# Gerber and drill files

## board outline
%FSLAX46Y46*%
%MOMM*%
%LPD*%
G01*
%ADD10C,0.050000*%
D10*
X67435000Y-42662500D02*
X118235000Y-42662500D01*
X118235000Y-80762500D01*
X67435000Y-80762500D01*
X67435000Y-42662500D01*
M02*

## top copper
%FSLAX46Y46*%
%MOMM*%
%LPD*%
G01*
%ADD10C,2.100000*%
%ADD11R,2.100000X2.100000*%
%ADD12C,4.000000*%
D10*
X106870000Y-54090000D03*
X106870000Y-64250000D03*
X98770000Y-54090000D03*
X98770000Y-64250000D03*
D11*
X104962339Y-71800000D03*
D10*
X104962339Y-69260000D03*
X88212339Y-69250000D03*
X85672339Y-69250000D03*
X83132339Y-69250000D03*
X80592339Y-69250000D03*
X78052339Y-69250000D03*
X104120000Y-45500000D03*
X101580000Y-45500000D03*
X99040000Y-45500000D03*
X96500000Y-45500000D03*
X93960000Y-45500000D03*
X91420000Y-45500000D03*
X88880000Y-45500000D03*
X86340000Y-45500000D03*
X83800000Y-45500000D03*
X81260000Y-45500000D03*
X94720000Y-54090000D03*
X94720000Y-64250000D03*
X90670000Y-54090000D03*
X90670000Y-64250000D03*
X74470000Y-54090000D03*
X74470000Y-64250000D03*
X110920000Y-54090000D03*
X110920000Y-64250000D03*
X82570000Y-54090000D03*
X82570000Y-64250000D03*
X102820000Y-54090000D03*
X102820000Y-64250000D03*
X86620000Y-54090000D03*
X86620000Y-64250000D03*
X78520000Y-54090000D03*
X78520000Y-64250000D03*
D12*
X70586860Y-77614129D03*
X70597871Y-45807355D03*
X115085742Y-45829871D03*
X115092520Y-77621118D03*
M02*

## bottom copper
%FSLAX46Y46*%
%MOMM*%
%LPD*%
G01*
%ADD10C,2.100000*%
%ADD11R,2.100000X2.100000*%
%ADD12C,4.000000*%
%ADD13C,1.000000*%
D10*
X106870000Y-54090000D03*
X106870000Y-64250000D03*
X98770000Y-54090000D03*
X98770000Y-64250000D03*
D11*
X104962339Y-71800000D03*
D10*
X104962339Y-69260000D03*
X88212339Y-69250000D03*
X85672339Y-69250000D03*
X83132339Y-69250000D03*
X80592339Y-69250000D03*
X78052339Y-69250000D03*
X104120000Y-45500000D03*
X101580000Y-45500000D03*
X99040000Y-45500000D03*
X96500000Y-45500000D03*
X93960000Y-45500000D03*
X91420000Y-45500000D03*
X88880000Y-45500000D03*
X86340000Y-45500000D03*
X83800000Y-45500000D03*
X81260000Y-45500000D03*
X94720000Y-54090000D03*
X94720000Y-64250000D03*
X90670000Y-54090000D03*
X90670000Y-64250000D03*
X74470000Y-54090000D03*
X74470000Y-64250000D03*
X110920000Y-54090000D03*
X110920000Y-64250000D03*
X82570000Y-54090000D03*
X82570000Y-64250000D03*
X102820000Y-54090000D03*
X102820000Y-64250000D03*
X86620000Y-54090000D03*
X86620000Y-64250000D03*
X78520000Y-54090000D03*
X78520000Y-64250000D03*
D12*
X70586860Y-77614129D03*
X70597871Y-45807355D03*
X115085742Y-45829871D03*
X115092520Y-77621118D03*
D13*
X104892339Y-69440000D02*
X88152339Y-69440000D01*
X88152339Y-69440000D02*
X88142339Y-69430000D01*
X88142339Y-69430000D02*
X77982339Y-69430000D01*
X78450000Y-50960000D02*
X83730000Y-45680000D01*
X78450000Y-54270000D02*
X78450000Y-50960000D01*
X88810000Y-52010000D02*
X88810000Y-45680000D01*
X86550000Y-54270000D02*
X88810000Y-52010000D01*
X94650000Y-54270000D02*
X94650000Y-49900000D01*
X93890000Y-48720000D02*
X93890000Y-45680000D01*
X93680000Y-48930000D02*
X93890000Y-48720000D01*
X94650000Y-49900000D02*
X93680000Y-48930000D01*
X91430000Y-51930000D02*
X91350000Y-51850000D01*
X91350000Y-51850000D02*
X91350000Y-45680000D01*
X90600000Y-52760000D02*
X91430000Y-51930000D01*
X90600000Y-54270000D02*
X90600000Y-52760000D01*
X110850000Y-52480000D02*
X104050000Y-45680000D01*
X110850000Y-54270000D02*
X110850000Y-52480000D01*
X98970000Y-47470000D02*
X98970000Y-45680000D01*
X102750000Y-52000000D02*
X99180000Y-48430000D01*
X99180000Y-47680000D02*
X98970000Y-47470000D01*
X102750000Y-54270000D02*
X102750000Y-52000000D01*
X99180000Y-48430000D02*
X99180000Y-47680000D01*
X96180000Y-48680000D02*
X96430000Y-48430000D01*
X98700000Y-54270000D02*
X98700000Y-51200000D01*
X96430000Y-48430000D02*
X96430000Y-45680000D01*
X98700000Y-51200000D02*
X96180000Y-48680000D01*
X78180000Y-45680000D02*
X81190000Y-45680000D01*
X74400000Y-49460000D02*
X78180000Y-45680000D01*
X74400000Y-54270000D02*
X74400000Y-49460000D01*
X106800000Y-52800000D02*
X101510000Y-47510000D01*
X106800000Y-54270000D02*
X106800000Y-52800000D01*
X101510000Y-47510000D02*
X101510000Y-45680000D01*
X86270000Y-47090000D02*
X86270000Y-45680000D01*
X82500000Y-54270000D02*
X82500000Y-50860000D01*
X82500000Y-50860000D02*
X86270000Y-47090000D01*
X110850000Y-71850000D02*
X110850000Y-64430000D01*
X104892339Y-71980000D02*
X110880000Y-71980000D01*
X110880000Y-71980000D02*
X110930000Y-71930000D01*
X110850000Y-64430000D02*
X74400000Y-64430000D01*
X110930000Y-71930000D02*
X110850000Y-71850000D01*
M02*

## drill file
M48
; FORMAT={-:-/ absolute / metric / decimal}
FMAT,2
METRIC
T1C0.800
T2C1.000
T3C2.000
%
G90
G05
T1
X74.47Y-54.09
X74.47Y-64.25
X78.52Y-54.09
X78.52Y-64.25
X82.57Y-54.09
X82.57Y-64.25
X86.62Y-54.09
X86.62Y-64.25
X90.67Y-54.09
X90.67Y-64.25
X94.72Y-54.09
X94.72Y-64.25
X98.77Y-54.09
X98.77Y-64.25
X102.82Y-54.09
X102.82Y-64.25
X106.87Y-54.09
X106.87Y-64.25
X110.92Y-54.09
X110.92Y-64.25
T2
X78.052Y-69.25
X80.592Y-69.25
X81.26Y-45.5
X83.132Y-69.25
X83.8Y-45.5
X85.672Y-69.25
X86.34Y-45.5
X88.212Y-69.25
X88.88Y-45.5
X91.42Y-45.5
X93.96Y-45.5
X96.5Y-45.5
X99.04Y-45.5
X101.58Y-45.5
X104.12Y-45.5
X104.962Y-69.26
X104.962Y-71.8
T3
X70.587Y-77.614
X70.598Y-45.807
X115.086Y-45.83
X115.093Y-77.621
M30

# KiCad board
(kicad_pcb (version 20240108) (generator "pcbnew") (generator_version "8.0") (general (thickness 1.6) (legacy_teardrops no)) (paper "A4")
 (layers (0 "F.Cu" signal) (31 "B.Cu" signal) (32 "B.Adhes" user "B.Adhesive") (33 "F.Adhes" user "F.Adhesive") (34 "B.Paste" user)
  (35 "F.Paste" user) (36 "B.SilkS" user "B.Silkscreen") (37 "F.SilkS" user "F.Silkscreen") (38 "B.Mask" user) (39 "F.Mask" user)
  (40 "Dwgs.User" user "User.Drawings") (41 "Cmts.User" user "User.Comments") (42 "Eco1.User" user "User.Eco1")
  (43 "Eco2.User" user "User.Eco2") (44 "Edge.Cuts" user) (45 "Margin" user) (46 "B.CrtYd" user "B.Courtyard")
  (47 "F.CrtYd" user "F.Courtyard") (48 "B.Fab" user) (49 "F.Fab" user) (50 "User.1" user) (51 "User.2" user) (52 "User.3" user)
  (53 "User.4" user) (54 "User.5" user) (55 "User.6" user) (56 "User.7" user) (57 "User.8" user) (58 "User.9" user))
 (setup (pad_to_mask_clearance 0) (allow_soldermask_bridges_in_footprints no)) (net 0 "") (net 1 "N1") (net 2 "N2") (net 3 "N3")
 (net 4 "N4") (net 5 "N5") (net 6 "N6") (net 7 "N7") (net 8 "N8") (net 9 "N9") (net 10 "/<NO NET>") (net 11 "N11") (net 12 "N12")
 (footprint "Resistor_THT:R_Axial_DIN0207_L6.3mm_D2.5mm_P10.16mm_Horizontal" (layer "F.Cu") (at 106.87 54.09 -90)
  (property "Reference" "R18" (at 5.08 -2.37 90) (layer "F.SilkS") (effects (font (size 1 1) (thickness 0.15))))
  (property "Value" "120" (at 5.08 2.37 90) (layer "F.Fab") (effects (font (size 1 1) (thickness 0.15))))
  (pad "1" thru_hole circle (at 0 0 270) (size 2.1 2.1) (drill 0.8) (layers "*.Cu" "*.Mask") (remove_unused_layers no) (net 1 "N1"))
  (pad "2" thru_hole circle (at 10.16 0 270) (size 2.1 2.1) (drill 0.8) (layers "*.Cu" "*.Mask") (remove_unused_layers no) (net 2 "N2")))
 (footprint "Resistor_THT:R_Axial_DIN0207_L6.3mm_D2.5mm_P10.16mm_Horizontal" (layer "F.Cu") (at 98.77 54.09 -90)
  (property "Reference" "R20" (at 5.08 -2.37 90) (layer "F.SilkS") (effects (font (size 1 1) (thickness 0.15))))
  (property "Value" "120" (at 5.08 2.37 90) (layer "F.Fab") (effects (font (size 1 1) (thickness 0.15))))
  (pad "1" thru_hole circle (at 0 0 270) (size 2.1 2.1) (drill 0.8) (layers "*.Cu" "*.Mask") (remove_unused_layers no) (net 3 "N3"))
  (pad "2" thru_hole circle (at 10.16 0 270) (size 2.1 2.1) (drill 0.8) (layers "*.Cu" "*.Mask") (remove_unused_layers no) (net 2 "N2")))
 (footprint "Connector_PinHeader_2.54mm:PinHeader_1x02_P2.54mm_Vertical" (layer "F.Cu") (at 104.962339 71.8 180)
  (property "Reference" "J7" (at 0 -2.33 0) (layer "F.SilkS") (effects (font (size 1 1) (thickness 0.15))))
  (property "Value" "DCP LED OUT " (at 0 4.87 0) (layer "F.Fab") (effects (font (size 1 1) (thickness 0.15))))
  (pad "1" thru_hole rect (at 0 0 180) (size 2.1 2.1) (drill 1) (layers "*.Cu" "*.Mask") (remove_unused_layers no) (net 2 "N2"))
  (pad "2" thru_hole circle (at 0 2.54 180) (size 2.1 2.1) (drill 1) (layers "*.Cu" "*.Mask") (remove_unused_layers no) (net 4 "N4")))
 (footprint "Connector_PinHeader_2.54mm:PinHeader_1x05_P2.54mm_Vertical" (layer "F.Cu") (at 88.212339 69.25 -90)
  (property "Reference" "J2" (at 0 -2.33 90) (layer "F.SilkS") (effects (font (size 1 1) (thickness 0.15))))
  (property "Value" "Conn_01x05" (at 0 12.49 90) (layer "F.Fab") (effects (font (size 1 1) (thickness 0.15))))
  (pad "1" thru_hole circle (at 0 0 270) (size 2.1 2.1) (drill 1) (layers "*.Cu" "*.Mask") (remove_unused_layers no) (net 4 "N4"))
  (pad "2" thru_hole circle (at 0 2.54 270) (size 2.1 2.1) (drill 1) (layers "*.Cu" "*.Mask") (remove_unused_layers no) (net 4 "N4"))
  (pad "3" thru_hole circle (at 0 5.08 270) (size 2.1 2.1) (drill 1) (layers "*.Cu" "*.Mask") (remove_unused_layers no) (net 4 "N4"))
  (pad "4" thru_hole circle (at 0 7.62 270) (size 2.1 2.1) (drill 1) (layers "*.Cu" "*.Mask") (remove_unused_layers no) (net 4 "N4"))
  (pad "5" thru_hole circle (at 0 10.16 270) (size 2.1 2.1) (drill 1) (layers "*.Cu" "*.Mask") (remove_unused_layers no) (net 4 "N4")))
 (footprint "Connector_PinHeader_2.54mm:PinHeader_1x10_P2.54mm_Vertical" (layer "F.Cu") (at 104.12 45.5 -90)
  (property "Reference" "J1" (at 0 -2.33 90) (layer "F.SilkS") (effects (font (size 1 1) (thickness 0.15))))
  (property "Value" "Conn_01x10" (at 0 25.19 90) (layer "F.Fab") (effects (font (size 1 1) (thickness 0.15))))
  (pad "1" thru_hole circle (at 0 0 270) (size 2.1 2.1) (drill 1) (layers "*.Cu" "*.Mask") (remove_unused_layers no) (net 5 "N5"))
  (pad "2" thru_hole circle (at 0 2.54 270) (size 2.1 2.1) (drill 1) (layers "*.Cu" "*.Mask") (remove_unused_layers no) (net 1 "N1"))
  (pad "3" thru_hole circle (at 0 5.08 270) (size 2.1 2.1) (drill 1) (layers "*.Cu" "*.Mask") (remove_unused_layers no) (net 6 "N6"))
  (pad "4" thru_hole circle (at 0 7.62 270) (size 2.1 2.1) (drill 1) (layers "*.Cu" "*.Mask") (remove_unused_layers no) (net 3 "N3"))
  (pad "5" thru_hole circle (at 0 10.16 270) (size 2.1 2.1) (drill 1) (layers "*.Cu" "*.Mask") (remove_unused_layers no) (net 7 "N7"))
  (pad "6" thru_hole circle (at 0 12.7 270) (size 2.1 2.1) (drill 1) (layers "*.Cu" "*.Mask") (remove_unused_layers no) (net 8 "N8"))
  (pad "7" thru_hole circle (at 0 15.24 270) (size 2.1 2.1) (drill 1) (layers "*.Cu" "*.Mask") (remove_unused_layers no) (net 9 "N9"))
  (pad "8" thru_hole circle (at 0 17.78 270) (size 2.1 2.1) (drill 1) (layers "*.Cu" "*.Mask") (remove_unused_layers no)
   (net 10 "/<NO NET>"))
  (pad "9" thru_hole circle (at 0 20.32 270) (size 2.1 2.1) (drill 1) (layers "*.Cu" "*.Mask") (remove_unused_layers no) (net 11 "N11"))
  (pad "10" thru_hole circle (at 0 22.86 270) (size 2.1 2.1) (drill 1) (layers "*.Cu" "*.Mask") (remove_unused_layers no) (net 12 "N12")))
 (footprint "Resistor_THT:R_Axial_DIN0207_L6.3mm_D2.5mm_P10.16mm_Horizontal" (layer "F.Cu") (at 94.72 54.09 -90)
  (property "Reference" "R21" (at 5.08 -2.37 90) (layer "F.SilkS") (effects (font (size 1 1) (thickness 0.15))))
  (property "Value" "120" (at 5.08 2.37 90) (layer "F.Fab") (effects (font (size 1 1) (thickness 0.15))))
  (pad "1" thru_hole circle (at 0 0 270) (size 2.1 2.1) (drill 0.8) (layers "*.Cu" "*.Mask") (remove_unused_layers no) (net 7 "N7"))
  (pad "2" thru_hole circle (at 10.16 0 270) (size 2.1 2.1) (drill 0.8) (layers "*.Cu" "*.Mask") (remove_unused_layers no) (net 2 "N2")))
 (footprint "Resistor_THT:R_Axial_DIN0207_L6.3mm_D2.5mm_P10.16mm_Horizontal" (layer "F.Cu") (at 90.67 54.09 -90)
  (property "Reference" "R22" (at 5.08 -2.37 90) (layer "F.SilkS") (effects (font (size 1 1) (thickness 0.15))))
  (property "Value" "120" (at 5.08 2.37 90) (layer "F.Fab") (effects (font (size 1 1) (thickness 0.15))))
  (pad "1" thru_hole circle (at 0 0 270) (size 2.1 2.1) (drill 0.8) (layers "*.Cu" "*.Mask") (remove_unused_layers no) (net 8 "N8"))
  (pad "2" thru_hole circle (at 10.16 0 270) (size 2.1 2.1) (drill 0.8) (layers "*.Cu" "*.Mask") (remove_unused_layers no) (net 2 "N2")))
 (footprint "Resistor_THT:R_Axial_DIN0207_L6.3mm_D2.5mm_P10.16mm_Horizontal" (layer "F.Cu") (at 74.47 54.09 -90)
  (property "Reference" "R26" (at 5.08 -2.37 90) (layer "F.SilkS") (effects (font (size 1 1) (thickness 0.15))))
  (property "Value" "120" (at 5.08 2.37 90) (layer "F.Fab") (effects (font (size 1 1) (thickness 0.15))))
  (pad "1" thru_hole circle (at 0 0 270) (size 2.1 2.1) (drill 0.8) (layers "*.Cu" "*.Mask") (remove_unused_layers no) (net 12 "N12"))
  (pad "2" thru_hole circle (at 10.16 0 270) (size 2.1 2.1) (drill 0.8) (layers "*.Cu" "*.Mask") (remove_unused_layers no) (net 2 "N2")))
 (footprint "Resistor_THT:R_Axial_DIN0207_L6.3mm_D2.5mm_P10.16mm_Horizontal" (layer "F.Cu") (at 110.92 54.09 -90)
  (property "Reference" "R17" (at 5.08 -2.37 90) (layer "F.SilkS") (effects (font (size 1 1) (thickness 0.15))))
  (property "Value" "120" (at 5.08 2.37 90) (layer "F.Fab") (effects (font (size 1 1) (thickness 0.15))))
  (pad "1" thru_hole circle (at 0 0 270) (size 2.1 2.1) (drill 0.8) (layers "*.Cu" "*.Mask") (remove_unused_layers no) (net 5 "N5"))
  (pad "2" thru_hole circle (at 10.16 0 270) (size 2.1 2.1) (drill 0.8) (layers "*.Cu" "*.Mask") (remove_unused_layers no) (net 2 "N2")))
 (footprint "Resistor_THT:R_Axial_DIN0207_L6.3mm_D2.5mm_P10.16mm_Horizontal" (layer "F.Cu") (at 82.57 54.09 -90)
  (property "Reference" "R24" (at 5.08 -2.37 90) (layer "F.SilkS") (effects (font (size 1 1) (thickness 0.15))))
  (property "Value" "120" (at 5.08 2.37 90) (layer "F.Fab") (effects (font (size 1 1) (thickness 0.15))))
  (pad "1" thru_hole circle (at 0 0 270) (size 2.1 2.1) (drill 0.8) (layers "*.Cu" "*.Mask") (remove_unused_layers no) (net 10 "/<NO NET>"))
  (pad "2" thru_hole circle (at 10.16 0 270) (size 2.1 2.1) (drill 0.8) (layers "*.Cu" "*.Mask") (remove_unused_layers no) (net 2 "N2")))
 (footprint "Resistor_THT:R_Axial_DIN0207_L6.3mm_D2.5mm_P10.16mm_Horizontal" (layer "F.Cu") (at 102.82 54.09 -90)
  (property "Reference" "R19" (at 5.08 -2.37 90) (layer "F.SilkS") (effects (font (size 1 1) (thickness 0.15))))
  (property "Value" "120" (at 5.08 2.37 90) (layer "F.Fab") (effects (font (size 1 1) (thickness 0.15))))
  (pad "1" thru_hole circle (at 0 0 270) (size 2.1 2.1) (drill 0.8) (layers "*.Cu" "*.Mask") (remove_unused_layers no) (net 6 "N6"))
  (pad "2" thru_hole circle (at 10.16 0 270) (size 2.1 2.1) (drill 0.8) (layers "*.Cu" "*.Mask") (remove_unused_layers no) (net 2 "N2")))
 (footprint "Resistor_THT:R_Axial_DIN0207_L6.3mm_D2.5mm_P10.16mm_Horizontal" (layer "F.Cu") (at 86.62 54.09 -90)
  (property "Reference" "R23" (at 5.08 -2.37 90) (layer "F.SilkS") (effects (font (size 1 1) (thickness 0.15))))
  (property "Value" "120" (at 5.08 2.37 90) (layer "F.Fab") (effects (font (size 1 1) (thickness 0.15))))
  (pad "1" thru_hole circle (at 0 0 270) (size 2.1 2.1) (drill 0.8) (layers "*.Cu" "*.Mask") (remove_unused_layers no) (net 9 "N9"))
  (pad "2" thru_hole circle (at 10.16 0 270) (size 2.1 2.1) (drill 0.8) (layers "*.Cu" "*.Mask") (remove_unused_layers no) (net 2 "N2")))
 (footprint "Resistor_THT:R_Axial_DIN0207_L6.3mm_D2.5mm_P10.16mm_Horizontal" (layer "F.Cu") (at 78.52 54.09 -90)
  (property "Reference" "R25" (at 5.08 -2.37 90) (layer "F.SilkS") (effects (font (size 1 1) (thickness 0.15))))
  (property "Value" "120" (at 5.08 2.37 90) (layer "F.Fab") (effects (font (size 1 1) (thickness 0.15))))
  (pad "1" thru_hole circle (at 0 0 270) (size 2.1 2.1) (drill 0.8) (layers "*.Cu" "*.Mask") (remove_unused_layers no) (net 11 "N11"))
  (pad "2" thru_hole circle (at 10.16 0 270) (size 2.1 2.1) (drill 0.8) (layers "*.Cu" "*.Mask") (remove_unused_layers no) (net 2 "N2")))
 (gr_rect (start 67.435 42.6625) (end 118.235 80.7625) (stroke (width 0.05) (type default)) (fill none) (layer "Edge.Cuts"))
 (via (at 70.58686 77.614129) (size 4) (drill 2) (layers "F.Cu" "B.Cu") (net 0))
 (via (at 70.597871 45.807355) (size 4) (drill 2) (layers "F.Cu" "B.Cu") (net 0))
 (via (at 115.085742 45.829871) (size 4) (drill 2) (layers "F.Cu" "B.Cu") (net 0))
 (via (at 115.09252 77.621118) (size 4) (drill 2) (layers "F.Cu" "B.Cu") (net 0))
 (segment (start 104.892339 69.44) (end 88.152339 69.44) (width 1) (layer "B.Cu") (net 4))
 (segment (start 88.152339 69.44) (end 88.142339 69.43) (width 1) (layer "B.Cu") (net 4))
 (segment (start 88.142339 69.43) (end 77.982339 69.43) (width 1) (layer "B.Cu") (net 4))
 (segment (start 78.45 50.96) (end 83.73 45.68) (width 1) (layer "B.Cu") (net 11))
 (segment (start 78.45 54.27) (end 78.45 50.96) (width 1) (layer "B.Cu") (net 11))
 (segment (start 88.81 52.01) (end 88.81 45.68) (width 1) (layer "B.Cu") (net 9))
 (segment (start 86.55 54.27) (end 88.81 52.01) (width 1) (layer "B.Cu") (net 9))
 (segment (start 94.65 54.27) (end 94.65 49.9) (width 1) (layer "B.Cu") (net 7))
 (segment (start 93.89 48.72) (end 93.89 45.68) (width 1) (layer "B.Cu") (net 7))
 (segment (start 93.68 48.93) (end 93.89 48.72) (width 1) (layer "B.Cu") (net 7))
 (segment (start 94.65 49.9) (end 93.68 48.93) (width 1) (layer "B.Cu") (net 7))
 (segment (start 91.43 51.93) (end 91.35 51.85) (width 1) (layer "B.Cu") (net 8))
 (segment (start 91.35 51.85) (end 91.35 45.68) (width 1) (layer "B.Cu") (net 8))
 (segment (start 90.6 52.76) (end 91.43 51.93) (width 1) (layer "B.Cu") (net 8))
 (segment (start 90.6 54.27) (end 90.6 52.76) (width 1) (layer "B.Cu") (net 8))
 (segment (start 110.85 52.48) (end 104.05 45.68) (width 1) (layer "B.Cu") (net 5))
 (segment (start 110.85 54.27) (end 110.85 52.48) (width 1) (layer "B.Cu") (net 5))
 (segment (start 98.97 47.47) (end 98.97 45.68) (width 1) (layer "B.Cu") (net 6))
 (segment (start 102.75 52) (end 99.18 48.43) (width 1) (layer "B.Cu") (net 6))
 (segment (start 99.18 47.68) (end 98.97 47.47) (width 1) (layer "B.Cu") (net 6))
 (segment (start 102.75 54.27) (end 102.75 52) (width 1) (layer "B.Cu") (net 6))
 (segment (start 99.18 48.43) (end 99.18 47.68) (width 1) (layer "B.Cu") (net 6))
 (segment (start 96.18 48.68) (end 96.43 48.43) (width 1) (layer "B.Cu") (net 3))
 (segment (start 98.7 54.27) (end 98.7 51.2) (width 1) (layer "B.Cu") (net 3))
 (segment (start 96.43 48.43) (end 96.43 45.68) (width 1) (layer "B.Cu") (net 3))
 (segment (start 98.7 51.2) (end 96.18 48.68) (width 1) (layer "B.Cu") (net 3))
 (segment (start 78.18 45.68) (end 81.19 45.68) (width 1) (layer "B.Cu") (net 12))
 (segment (start 74.4 49.46) (end 78.18 45.68) (width 1) (layer "B.Cu") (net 12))
 (segment (start 74.4 54.27) (end 74.4 49.46) (width 1) (layer "B.Cu") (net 12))
 (segment (start 106.8 52.8) (end 101.51 47.51) (width 1) (layer "B.Cu") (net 1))
 (segment (start 106.8 54.27) (end 106.8 52.8) (width 1) (layer "B.Cu") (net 1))
 (segment (start 101.51 47.51) (end 101.51 45.68) (width 1) (layer "B.Cu") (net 1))
 (segment (start 86.27 47.09) (end 86.27 45.68) (width 1) (layer "B.Cu") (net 10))
 (segment (start 82.5 54.27) (end 82.5 50.86) (width 1) (layer "B.Cu") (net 10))
 (segment (start 82.5 50.86) (end 86.27 47.09) (width 1) (layer "B.Cu") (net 10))
 (segment (start 110.85 71.85) (end 110.85 64.43) (width 1) (layer "B.Cu") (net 2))
 (segment (start 104.892339 71.98) (end 110.88 71.98) (width 1) (layer "B.Cu") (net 2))
 (segment (start 110.88 71.98) (end 110.93 71.93) (width 1) (layer "B.Cu") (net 2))
 (segment (start 110.85 64.43) (end 74.4 64.43) (width 1) (layer "B.Cu") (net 2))
 (segment (start 110.93 71.93) (end 110.85 71.85) (width 1) (layer "B.Cu") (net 2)))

